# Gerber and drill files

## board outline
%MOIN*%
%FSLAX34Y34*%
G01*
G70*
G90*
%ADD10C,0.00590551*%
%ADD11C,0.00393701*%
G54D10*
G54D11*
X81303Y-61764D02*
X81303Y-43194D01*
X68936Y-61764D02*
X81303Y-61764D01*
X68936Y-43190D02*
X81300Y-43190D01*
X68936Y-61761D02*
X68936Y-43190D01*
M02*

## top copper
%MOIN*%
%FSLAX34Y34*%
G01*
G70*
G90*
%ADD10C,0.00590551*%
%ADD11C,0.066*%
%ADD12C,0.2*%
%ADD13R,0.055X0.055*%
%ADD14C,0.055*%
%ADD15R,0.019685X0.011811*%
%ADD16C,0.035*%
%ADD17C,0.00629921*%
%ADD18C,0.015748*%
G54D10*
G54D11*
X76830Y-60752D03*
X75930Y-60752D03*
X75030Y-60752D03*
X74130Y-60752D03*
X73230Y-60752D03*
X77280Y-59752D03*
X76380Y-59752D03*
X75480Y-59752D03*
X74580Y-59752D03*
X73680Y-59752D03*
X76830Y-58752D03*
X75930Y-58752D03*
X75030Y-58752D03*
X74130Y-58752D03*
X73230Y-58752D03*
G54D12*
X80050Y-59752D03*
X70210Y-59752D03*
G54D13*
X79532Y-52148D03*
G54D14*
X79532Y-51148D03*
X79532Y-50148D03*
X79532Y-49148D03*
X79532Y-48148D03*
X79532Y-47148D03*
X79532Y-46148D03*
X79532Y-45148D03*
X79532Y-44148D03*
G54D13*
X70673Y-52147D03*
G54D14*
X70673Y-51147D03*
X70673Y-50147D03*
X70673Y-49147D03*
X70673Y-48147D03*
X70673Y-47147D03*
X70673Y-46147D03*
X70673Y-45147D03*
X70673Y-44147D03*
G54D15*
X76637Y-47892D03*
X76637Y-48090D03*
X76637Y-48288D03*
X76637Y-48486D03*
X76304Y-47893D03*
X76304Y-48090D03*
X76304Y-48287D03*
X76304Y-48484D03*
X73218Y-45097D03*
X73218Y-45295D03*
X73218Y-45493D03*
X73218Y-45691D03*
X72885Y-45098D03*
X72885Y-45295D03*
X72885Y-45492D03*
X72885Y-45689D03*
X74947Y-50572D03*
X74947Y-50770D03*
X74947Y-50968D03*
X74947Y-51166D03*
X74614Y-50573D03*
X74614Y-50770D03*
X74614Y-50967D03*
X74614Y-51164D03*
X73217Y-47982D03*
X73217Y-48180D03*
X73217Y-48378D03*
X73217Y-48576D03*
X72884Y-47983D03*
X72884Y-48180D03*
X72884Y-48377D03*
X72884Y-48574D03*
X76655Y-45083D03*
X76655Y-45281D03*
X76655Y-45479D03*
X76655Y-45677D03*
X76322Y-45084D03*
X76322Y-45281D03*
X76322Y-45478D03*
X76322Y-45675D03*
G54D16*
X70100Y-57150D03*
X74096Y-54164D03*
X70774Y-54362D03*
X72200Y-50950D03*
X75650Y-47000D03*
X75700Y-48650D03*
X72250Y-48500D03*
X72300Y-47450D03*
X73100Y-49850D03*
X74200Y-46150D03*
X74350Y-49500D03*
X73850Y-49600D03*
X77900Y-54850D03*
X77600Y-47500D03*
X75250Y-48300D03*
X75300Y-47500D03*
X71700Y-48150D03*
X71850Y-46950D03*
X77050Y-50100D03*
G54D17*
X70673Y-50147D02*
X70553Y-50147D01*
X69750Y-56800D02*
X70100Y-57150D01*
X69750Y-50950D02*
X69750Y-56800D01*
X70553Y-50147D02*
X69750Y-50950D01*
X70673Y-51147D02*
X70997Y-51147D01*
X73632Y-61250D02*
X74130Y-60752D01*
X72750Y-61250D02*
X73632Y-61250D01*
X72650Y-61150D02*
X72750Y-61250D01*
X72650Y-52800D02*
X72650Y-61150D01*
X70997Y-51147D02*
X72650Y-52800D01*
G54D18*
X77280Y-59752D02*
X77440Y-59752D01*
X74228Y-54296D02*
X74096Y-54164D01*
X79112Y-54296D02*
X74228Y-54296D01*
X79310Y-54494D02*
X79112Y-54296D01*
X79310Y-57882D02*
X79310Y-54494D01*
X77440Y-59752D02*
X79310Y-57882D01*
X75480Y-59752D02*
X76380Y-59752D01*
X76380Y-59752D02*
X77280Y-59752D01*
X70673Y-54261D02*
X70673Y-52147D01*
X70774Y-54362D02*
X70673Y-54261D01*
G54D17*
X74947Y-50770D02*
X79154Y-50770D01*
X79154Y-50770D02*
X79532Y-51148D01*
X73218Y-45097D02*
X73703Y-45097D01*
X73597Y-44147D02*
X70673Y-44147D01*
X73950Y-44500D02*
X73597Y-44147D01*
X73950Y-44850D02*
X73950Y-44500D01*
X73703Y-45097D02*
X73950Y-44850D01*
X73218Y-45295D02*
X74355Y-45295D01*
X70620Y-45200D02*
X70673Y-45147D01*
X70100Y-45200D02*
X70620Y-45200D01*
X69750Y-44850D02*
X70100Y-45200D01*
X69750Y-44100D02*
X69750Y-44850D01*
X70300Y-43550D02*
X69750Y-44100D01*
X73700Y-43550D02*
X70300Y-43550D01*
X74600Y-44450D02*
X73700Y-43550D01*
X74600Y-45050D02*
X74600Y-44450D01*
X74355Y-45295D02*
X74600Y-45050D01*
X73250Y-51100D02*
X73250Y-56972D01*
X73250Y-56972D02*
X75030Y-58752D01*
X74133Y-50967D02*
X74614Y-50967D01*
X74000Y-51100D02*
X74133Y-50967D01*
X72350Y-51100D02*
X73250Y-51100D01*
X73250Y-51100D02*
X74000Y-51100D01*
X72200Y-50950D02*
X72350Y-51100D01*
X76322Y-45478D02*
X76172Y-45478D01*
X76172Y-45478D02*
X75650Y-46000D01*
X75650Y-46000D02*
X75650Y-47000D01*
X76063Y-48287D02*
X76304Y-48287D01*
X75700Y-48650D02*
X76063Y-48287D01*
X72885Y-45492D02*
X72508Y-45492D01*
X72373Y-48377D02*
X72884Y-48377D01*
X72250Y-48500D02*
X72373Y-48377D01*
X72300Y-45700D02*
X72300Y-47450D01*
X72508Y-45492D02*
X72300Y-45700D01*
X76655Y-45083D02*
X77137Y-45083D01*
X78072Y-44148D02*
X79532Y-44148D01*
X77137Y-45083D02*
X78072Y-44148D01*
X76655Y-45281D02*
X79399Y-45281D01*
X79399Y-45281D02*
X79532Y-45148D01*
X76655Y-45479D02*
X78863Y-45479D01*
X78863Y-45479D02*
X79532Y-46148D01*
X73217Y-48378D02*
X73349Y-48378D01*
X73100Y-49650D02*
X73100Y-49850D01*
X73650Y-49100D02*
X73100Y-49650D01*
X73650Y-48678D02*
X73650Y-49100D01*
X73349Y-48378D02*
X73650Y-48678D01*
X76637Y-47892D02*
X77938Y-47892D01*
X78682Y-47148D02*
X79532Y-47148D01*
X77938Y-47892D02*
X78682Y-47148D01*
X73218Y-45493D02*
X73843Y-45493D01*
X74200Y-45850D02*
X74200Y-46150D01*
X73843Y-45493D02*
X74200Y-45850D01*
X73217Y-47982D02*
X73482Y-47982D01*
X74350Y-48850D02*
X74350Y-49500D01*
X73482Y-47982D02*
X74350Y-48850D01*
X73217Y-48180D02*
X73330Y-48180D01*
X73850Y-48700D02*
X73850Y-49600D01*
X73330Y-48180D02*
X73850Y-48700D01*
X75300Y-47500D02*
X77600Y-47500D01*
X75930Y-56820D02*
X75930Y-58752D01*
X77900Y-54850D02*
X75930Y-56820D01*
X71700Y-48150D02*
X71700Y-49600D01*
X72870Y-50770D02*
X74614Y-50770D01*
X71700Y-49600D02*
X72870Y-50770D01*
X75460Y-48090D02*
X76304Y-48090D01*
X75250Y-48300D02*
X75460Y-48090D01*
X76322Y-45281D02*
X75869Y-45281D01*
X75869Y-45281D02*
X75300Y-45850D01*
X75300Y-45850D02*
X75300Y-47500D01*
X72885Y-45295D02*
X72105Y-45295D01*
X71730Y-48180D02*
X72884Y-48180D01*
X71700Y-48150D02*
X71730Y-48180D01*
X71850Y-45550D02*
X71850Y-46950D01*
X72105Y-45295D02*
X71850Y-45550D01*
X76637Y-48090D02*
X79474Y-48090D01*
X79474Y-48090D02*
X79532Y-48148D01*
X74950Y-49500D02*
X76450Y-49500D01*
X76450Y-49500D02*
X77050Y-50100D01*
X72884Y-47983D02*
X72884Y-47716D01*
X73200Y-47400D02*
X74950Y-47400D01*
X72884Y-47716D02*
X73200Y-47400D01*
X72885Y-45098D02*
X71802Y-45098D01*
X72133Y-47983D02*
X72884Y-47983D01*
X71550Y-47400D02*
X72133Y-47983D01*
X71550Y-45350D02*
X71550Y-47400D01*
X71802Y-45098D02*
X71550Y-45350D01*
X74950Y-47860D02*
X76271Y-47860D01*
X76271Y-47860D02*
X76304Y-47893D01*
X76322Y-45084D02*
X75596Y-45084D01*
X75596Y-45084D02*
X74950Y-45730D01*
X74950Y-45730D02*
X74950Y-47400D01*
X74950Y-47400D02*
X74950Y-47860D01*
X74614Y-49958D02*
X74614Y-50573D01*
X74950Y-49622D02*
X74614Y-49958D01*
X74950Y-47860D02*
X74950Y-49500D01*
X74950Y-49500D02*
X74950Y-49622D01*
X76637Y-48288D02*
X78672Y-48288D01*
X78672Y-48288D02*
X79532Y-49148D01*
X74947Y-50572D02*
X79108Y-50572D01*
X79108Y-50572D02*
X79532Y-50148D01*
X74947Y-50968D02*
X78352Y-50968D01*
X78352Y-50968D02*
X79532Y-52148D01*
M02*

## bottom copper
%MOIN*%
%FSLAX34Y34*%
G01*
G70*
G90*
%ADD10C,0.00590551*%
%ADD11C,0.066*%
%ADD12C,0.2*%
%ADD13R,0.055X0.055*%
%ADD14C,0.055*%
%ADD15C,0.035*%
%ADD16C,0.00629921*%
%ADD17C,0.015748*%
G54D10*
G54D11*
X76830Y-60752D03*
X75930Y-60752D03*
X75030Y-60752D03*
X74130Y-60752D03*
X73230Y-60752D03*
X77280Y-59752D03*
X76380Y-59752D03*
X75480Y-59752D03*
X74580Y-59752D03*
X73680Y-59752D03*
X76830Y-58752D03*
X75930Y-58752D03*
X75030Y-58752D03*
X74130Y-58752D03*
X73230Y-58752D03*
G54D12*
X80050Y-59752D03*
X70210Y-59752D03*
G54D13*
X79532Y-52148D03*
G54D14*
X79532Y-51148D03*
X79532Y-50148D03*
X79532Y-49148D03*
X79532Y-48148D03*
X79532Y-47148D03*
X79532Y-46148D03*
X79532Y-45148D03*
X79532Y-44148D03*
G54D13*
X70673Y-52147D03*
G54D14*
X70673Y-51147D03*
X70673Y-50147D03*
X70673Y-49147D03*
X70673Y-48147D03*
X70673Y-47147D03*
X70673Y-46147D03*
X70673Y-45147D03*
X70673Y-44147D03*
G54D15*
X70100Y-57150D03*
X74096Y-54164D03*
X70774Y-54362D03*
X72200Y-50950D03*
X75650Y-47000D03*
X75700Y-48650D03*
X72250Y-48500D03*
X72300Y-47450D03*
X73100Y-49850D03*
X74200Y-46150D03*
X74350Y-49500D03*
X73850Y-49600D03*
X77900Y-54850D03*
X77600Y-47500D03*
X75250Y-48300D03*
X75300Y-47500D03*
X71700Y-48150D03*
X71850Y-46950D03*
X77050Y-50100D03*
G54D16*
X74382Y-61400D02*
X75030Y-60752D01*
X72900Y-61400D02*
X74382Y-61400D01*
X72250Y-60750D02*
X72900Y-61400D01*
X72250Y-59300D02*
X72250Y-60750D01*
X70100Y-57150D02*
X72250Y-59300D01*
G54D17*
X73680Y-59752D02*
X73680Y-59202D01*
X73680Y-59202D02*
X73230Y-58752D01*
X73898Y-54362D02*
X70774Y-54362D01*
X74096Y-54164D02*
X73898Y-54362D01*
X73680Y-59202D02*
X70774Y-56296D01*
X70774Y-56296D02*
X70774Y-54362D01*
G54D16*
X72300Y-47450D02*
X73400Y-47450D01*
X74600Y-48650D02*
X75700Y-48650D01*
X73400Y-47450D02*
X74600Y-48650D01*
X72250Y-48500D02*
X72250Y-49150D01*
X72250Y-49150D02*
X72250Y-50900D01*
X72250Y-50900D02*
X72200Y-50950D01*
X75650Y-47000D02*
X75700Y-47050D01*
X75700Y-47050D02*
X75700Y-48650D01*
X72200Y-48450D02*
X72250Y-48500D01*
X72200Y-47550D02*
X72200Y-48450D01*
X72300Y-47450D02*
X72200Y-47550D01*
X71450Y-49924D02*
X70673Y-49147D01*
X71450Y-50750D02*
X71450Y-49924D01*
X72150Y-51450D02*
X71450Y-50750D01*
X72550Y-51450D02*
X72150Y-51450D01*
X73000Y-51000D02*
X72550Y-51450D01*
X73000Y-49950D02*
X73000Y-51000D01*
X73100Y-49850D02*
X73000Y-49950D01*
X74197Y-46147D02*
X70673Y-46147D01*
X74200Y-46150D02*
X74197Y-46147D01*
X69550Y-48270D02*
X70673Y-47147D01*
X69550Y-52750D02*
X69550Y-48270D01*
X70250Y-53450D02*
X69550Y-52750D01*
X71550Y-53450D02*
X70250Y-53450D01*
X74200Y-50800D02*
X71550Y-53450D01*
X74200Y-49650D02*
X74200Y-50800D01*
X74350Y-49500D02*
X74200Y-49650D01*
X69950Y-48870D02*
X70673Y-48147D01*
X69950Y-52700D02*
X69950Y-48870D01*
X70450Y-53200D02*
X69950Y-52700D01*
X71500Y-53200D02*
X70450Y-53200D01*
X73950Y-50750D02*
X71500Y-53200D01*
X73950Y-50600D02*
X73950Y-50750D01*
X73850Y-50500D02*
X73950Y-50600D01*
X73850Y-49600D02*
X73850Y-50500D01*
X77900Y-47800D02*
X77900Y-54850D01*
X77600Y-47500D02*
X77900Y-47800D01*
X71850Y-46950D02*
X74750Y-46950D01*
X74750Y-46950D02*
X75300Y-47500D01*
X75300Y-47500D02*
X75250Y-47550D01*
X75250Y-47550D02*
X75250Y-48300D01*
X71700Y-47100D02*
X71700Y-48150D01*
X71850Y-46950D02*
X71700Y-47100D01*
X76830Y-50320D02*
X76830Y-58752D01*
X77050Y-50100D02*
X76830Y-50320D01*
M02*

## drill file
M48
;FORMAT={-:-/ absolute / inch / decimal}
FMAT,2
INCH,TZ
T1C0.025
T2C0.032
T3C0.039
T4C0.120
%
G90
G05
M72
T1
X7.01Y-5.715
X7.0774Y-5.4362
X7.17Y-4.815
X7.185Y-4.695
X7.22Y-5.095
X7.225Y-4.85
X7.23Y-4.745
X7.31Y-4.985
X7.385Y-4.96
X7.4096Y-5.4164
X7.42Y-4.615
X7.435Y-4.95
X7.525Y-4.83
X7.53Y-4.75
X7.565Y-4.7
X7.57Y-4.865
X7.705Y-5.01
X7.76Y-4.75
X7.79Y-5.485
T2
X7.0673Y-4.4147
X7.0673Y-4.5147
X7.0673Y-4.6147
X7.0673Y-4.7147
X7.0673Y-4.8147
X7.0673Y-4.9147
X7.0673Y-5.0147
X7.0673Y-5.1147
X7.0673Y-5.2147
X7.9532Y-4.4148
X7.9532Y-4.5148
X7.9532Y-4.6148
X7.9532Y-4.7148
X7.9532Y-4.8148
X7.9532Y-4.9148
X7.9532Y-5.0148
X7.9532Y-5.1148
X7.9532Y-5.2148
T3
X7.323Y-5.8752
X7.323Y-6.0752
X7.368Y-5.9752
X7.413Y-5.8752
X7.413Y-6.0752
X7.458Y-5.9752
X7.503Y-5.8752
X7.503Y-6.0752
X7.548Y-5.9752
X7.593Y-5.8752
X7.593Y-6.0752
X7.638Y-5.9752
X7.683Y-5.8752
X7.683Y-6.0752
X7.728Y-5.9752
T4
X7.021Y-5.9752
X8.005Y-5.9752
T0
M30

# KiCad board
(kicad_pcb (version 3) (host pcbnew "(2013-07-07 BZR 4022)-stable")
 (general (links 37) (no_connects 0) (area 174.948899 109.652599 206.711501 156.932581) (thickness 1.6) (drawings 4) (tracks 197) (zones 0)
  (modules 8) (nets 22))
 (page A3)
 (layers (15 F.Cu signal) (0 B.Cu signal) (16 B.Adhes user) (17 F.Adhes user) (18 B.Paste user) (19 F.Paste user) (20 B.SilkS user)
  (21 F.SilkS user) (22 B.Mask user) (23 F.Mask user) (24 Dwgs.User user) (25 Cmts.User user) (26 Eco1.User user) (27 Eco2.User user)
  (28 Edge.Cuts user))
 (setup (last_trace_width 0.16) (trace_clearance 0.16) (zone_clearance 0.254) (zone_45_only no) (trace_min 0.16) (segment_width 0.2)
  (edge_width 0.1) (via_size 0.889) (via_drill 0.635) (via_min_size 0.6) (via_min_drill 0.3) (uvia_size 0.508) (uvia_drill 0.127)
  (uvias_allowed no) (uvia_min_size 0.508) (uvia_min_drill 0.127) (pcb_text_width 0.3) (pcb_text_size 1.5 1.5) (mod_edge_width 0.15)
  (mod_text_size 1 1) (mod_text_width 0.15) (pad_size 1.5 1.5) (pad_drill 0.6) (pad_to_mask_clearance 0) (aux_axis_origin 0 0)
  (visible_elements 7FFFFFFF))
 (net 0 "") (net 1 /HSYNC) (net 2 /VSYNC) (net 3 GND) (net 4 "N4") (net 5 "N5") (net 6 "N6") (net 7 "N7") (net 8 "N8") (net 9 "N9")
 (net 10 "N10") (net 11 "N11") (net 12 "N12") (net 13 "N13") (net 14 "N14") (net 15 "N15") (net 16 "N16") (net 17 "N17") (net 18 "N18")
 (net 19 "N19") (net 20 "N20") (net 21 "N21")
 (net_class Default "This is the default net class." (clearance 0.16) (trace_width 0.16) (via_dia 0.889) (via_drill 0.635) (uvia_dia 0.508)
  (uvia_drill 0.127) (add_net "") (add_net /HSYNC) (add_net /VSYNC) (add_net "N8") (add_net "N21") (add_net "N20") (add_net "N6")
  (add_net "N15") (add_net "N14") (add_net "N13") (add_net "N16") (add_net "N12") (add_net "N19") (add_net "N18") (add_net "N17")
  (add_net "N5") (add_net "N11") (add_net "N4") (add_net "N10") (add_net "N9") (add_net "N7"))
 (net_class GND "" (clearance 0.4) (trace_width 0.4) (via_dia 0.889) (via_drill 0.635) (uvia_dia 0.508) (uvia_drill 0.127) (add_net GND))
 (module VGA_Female (layer F.Cu) (at 190.8302 151.77008)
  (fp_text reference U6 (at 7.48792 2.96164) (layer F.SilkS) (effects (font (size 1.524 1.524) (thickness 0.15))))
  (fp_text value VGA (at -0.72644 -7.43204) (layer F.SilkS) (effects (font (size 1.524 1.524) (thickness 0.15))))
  (pad 11 thru_hole circle (at 4.318 2.54) (size 1.6764 1.6764) (drill 0.9906) (layers *.Cu F.Paste F.SilkS F.Mask))
  (pad 12 thru_hole circle (at 2.032 2.54) (size 1.6764 1.6764) (drill 0.9906) (layers *.Cu F.Paste F.SilkS F.Mask))
  (pad 13 thru_hole circle (at -0.254 2.54) (size 1.6764 1.6764) (drill 0.9906) (layers *.Cu F.Paste F.SilkS F.Mask) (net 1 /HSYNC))
  (pad 14 thru_hole circle (at -2.54 2.54) (size 1.6764 1.6764) (drill 0.9906) (layers *.Cu F.Paste F.SilkS F.Mask) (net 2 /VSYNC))
  (pad 15 thru_hole circle (at -4.826 2.54) (size 1.6764 1.6764) (drill 0.9906) (layers *.Cu F.Paste F.SilkS F.Mask))
  (pad 6 thru_hole circle (at 5.461 0) (size 1.6764 1.6764) (drill 0.9906) (layers *.Cu F.Paste F.SilkS F.Mask) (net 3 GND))
  (pad 7 thru_hole circle (at 3.175 0) (size 1.6764 1.6764) (drill 0.9906) (layers *.Cu F.Paste F.SilkS F.Mask) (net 3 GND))
  (pad 8 thru_hole circle (at 0.889 0) (size 1.6764 1.6764) (drill 0.9906) (layers *.Cu F.Paste F.SilkS F.Mask) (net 3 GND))
  (pad 9 thru_hole circle (at -1.397 0) (size 1.6764 1.6764) (drill 0.9906) (layers *.Cu F.Paste F.SilkS F.Mask))
  (pad 10 thru_hole circle (at -3.683 0) (size 1.6764 1.6764) (drill 0.9906) (layers *.Cu F.Paste F.SilkS F.Mask) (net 3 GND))
  (pad 1 thru_hole circle (at 4.318 -2.54) (size 1.6764 1.6764) (drill 0.9906) (layers *.Cu F.Paste F.SilkS F.Mask) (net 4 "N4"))
  (pad 2 thru_hole circle (at 2.032 -2.54) (size 1.6764 1.6764) (drill 0.9906) (layers *.Cu F.Paste F.SilkS F.Mask) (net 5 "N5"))
  (pad 3 thru_hole circle (at -0.254 -2.54) (size 1.6764 1.6764) (drill 0.9906) (layers *.Cu F.Paste F.SilkS F.Mask) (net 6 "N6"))
  (pad 4 thru_hole circle (at -2.54 -2.54) (size 1.6764 1.6764) (drill 0.9906) (layers *.Cu F.Paste F.SilkS F.Mask))
  (pad 5 thru_hole circle (at -4.826 -2.54) (size 1.6764 1.6764) (drill 0.9906) (layers *.Cu F.Paste F.SilkS F.Mask) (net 3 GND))
  (pad SH1 thru_hole circle (at 12.4968 0) (size 5.08 5.08) (drill 3.048) (layers *.Cu F.Paste F.SilkS F.Mask))
  (pad SH2 thru_hole circle (at -12.4968 0) (size 5.08 5.08) (drill 3.048) (layers *.Cu F.Paste F.SilkS F.Mask)))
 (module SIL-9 (layer F.Cu) (at 202.01128 122.29592 90)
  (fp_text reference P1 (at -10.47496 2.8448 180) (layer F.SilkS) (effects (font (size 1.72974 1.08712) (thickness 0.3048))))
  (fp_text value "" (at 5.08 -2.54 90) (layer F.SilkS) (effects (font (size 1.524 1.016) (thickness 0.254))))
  (pad 1 thru_hole rect (at -10.16 0 90) (size 1.397 1.397) (drill 0.8128) (layers *.Cu *.Mask F.SilkS) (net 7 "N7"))
  (pad 2 thru_hole circle (at -7.62 0 90) (size 1.397 1.397) (drill 0.8128) (layers *.Cu *.Mask F.SilkS) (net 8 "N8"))
  (pad 3 thru_hole circle (at -5.08 0 90) (size 1.397 1.397) (drill 0.8128) (layers *.Cu *.Mask F.SilkS) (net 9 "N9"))
  (pad 4 thru_hole circle (at -2.54 0 90) (size 1.397 1.397) (drill 0.8128) (layers *.Cu *.Mask F.SilkS) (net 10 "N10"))
  (pad 5 thru_hole circle (at 0 0 90) (size 1.397 1.397) (drill 0.8128) (layers *.Cu *.Mask F.SilkS) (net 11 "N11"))
  (pad 6 thru_hole circle (at 2.54 0 90) (size 1.397 1.397) (drill 0.8128) (layers *.Cu *.Mask F.SilkS) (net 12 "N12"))
  (pad 7 thru_hole circle (at 5.08 0 90) (size 1.397 1.397) (drill 0.8128) (layers *.Cu *.Mask F.SilkS) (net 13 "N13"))
  (pad 8 thru_hole circle (at 7.62 0 90) (size 1.397 1.397) (drill 0.8128) (layers *.Cu *.Mask F.SilkS) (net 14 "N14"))
  (pad 9 thru_hole circle (at 10.16 0 90) (size 1.397 1.397) (drill 0.8128) (layers *.Cu *.Mask F.SilkS) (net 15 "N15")))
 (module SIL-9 (layer F.Cu) (at 179.50942 122.29338 90)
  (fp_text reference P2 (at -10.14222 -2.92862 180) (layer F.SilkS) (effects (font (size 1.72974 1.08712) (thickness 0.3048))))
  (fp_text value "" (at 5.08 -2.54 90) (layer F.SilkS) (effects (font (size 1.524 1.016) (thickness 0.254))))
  (pad 1 thru_hole rect (at -10.16 0 90) (size 1.397 1.397) (drill 0.8128) (layers *.Cu *.Mask F.SilkS) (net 3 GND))
  (pad 2 thru_hole circle (at -7.62 0 90) (size 1.397 1.397) (drill 0.8128) (layers *.Cu *.Mask F.SilkS) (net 2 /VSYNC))
  (pad 3 thru_hole circle (at -5.08 0 90) (size 1.397 1.397) (drill 0.8128) (layers *.Cu *.Mask F.SilkS) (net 1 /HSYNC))
  (pad 4 thru_hole circle (at -2.54 0 90) (size 1.397 1.397) (drill 0.8128) (layers *.Cu *.Mask F.SilkS) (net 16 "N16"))
  (pad 5 thru_hole circle (at 0 0 90) (size 1.397 1.397) (drill 0.8128) (layers *.Cu *.Mask F.SilkS) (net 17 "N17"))
  (pad 6 thru_hole circle (at 2.54 0 90) (size 1.397 1.397) (drill 0.8128) (layers *.Cu *.Mask F.SilkS) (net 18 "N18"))
  (pad 7 thru_hole circle (at 5.08 0 90) (size 1.397 1.397) (drill 0.8128) (layers *.Cu *.Mask F.SilkS) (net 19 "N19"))
  (pad 8 thru_hole circle (at 7.62 0 90) (size 1.397 1.397) (drill 0.8128) (layers *.Cu *.Mask F.SilkS) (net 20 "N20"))
  (pad 9 thru_hole circle (at 10.16 0 90) (size 1.397 1.397) (drill 0.8128) (layers *.Cu *.Mask F.SilkS) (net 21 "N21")))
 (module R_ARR (layer F.Cu) (at 195.6943 122.3137 270)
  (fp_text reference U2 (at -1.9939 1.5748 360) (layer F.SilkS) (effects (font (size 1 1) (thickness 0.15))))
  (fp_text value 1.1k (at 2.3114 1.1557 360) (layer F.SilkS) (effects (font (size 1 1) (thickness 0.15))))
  (pad 1 smd rect (at -0.66802 1.03632 90) (size 0.3 0.5) (layers F.Cu F.Paste F.Mask) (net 12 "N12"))
  (pad 2 smd rect (at -0.1651 1.03632 90) (size 0.3 0.5) (layers F.Cu F.Paste F.Mask) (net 11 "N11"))
  (pad 3 smd rect (at 0.33782 1.03632 90) (size 0.3 0.5) (layers F.Cu F.Paste F.Mask) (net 10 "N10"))
  (pad 4 smd rect (at 0.84074 1.03632 90) (size 0.3 0.5) (layers F.Cu F.Paste F.Mask))
  (pad 5 smd rect (at -0.66548 1.88214 90) (size 0.3 0.5) (layers F.Cu F.Paste F.Mask) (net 4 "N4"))
  (pad 6 smd rect (at -0.1651 1.88214 90) (size 0.3 0.5) (layers F.Cu F.Paste F.Mask) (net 5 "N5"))
  (pad 7 smd rect (at 0.33528 1.88214 90) (size 0.3 0.5) (layers F.Cu F.Paste F.Mask) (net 6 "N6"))
  (pad 8 smd rect (at 0.83566 1.88214 90) (size 0.3 0.5) (layers F.Cu F.Paste F.Mask)))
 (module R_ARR (layer F.Cu) (at 187.01004 115.2144 270)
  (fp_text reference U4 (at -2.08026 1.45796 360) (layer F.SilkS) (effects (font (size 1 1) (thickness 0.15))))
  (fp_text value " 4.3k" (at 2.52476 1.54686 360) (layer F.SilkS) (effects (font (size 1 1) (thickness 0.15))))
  (pad 1 smd rect (at -0.66802 1.03632 90) (size 0.3 0.5) (layers F.Cu F.Paste F.Mask) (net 21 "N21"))
  (pad 2 smd rect (at -0.1651 1.03632 90) (size 0.3 0.5) (layers F.Cu F.Paste F.Mask) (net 20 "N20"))
  (pad 3 smd rect (at 0.33782 1.03632 90) (size 0.3 0.5) (layers F.Cu F.Paste F.Mask) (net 19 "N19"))
  (pad 4 smd rect (at 0.84074 1.03632 90) (size 0.3 0.5) (layers F.Cu F.Paste F.Mask))
  (pad 5 smd rect (at -0.66548 1.88214 90) (size 0.3 0.5) (layers F.Cu F.Paste F.Mask) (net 4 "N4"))
  (pad 6 smd rect (at -0.1651 1.88214 90) (size 0.3 0.5) (layers F.Cu F.Paste F.Mask) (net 5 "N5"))
  (pad 7 smd rect (at 0.33528 1.88214 90) (size 0.3 0.5) (layers F.Cu F.Paste F.Mask) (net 6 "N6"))
  (pad 8 smd rect (at 0.83566 1.88214 90) (size 0.3 0.5) (layers F.Cu F.Paste F.Mask)))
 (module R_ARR (layer F.Cu) (at 191.4017 129.1209 270)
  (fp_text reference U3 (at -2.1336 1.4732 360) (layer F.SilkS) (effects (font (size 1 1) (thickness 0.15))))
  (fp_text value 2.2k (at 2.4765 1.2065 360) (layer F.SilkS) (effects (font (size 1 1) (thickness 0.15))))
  (pad 1 smd rect (at -0.66802 1.03632 90) (size 0.3 0.5) (layers F.Cu F.Paste F.Mask) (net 9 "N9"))
  (pad 2 smd rect (at -0.1651 1.03632 90) (size 0.3 0.5) (layers F.Cu F.Paste F.Mask) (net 8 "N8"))
  (pad 3 smd rect (at 0.33782 1.03632 90) (size 0.3 0.5) (layers F.Cu F.Paste F.Mask) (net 7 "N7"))
  (pad 4 smd rect (at 0.84074 1.03632 90) (size 0.3 0.5) (layers F.Cu F.Paste F.Mask))
  (pad 5 smd rect (at -0.66548 1.88214 90) (size 0.3 0.5) (layers F.Cu F.Paste F.Mask) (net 4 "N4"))
  (pad 6 smd rect (at -0.1651 1.88214 90) (size 0.3 0.5) (layers F.Cu F.Paste F.Mask) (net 5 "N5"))
  (pad 7 smd rect (at 0.33528 1.88214 90) (size 0.3 0.5) (layers F.Cu F.Paste F.Mask) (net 6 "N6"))
  (pad 8 smd rect (at 0.83566 1.88214 90) (size 0.3 0.5) (layers F.Cu F.Paste F.Mask)))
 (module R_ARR (layer F.Cu) (at 187.0075 122.5423 270)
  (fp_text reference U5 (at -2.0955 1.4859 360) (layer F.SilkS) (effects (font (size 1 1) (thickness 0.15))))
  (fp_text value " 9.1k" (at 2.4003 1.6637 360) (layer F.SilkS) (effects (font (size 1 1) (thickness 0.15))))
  (pad 1 smd rect (at -0.66802 1.03632 90) (size 0.3 0.5) (layers F.Cu F.Paste F.Mask) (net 18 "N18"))
  (pad 2 smd rect (at -0.1651 1.03632 90) (size 0.3 0.5) (layers F.Cu F.Paste F.Mask) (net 17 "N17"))
  (pad 3 smd rect (at 0.33782 1.03632 90) (size 0.3 0.5) (layers F.Cu F.Paste F.Mask) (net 16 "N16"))
  (pad 4 smd rect (at 0.84074 1.03632 90) (size 0.3 0.5) (layers F.Cu F.Paste F.Mask))
  (pad 5 smd rect (at -0.66548 1.88214 90) (size 0.3 0.5) (layers F.Cu F.Paste F.Mask) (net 4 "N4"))
  (pad 6 smd rect (at -0.1651 1.88214 90) (size 0.3 0.5) (layers F.Cu F.Paste F.Mask) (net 5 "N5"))
  (pad 7 smd rect (at 0.33528 1.88214 90) (size 0.3 0.5) (layers F.Cu F.Paste F.Mask) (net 6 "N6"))
  (pad 8 smd rect (at 0.83566 1.88214 90) (size 0.3 0.5) (layers F.Cu F.Paste F.Mask)))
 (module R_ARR (layer F.Cu) (at 195.74002 115.17884 270)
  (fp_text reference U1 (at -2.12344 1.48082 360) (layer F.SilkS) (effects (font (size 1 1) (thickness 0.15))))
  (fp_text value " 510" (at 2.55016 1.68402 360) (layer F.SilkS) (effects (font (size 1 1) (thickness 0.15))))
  (pad 1 smd rect (at -0.66802 1.03632 90) (size 0.3 0.5) (layers F.Cu F.Paste F.Mask) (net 15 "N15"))
  (pad 2 smd rect (at -0.1651 1.03632 90) (size 0.3 0.5) (layers F.Cu F.Paste F.Mask) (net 14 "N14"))
  (pad 3 smd rect (at 0.33782 1.03632 90) (size 0.3 0.5) (layers F.Cu F.Paste F.Mask) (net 13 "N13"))
  (pad 4 smd rect (at 0.84074 1.03632 90) (size 0.3 0.5) (layers F.Cu F.Paste F.Mask))
  (pad 5 smd rect (at -0.66548 1.88214 90) (size 0.3 0.5) (layers F.Cu F.Paste F.Mask) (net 4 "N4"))
  (pad 6 smd rect (at -0.1651 1.88214 90) (size 0.3 0.5) (layers F.Cu F.Paste F.Mask) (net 5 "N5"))
  (pad 7 smd rect (at 0.33528 1.88214 90) (size 0.3 0.5) (layers F.Cu F.Paste F.Mask) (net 6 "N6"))
  (pad 8 smd rect (at 0.83566 1.88214 90) (size 0.3 0.5) (layers F.Cu F.Paste F.Mask)))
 (gr_line (start 206.50962 156.88056) (end 206.50962 109.71276) (angle 90) (layer Edge.Cuts) (width 0.1))
 (gr_line (start 175.09744 156.88056) (end 206.50962 156.88056) (angle 90) (layer Edge.Cuts) (width 0.1))
 (gr_line (start 175.09744 109.7026) (end 206.502 109.7026) (angle 90) (layer Edge.Cuts) (width 0.1))
 (gr_line (start 175.09744 156.87294) (end 175.09744 109.7026) (angle 90) (layer Edge.Cuts) (width 0.1))
 (segment (start 179.50942 127.37338) (end 179.20462 127.37338) (width 0.16) (layer F.Cu) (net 1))
 (segment (start 188.93028 155.956) (end 190.5762 154.31008) (width 0.16) (layer B.Cu) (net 1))
 (segment (start 185.166 155.956) (end 188.93028 155.956) (width 0.16) (layer B.Cu) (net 1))
 (segment (start 183.515 154.305) (end 185.166 155.956) (width 0.16) (layer B.Cu) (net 1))
 (segment (start 183.515 150.622) (end 183.515 154.305) (width 0.16) (layer B.Cu) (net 1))
 (segment (start 178.054 145.161) (end 183.515 150.622) (width 0.16) (layer B.Cu) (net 1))
 (via (at 178.054 145.161) (size 0.889) (layers F.Cu B.Cu) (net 1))
 (segment (start 177.165 144.272) (end 178.054 145.161) (width 0.16) (layer F.Cu) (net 1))
 (segment (start 177.165 129.413) (end 177.165 144.272) (width 0.16) (layer F.Cu) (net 1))
 (segment (start 179.20462 127.37338) (end 177.165 129.413) (width 0.16) (layer F.Cu) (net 1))
 (segment (start 179.50942 129.91338) (end 180.33238 129.91338) (width 0.16) (layer F.Cu) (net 2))
 (segment (start 187.02528 155.575) (end 188.2902 154.31008) (width 0.16) (layer F.Cu) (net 2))
 (segment (start 184.785 155.575) (end 187.02528 155.575) (width 0.16) (layer F.Cu) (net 2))
 (segment (start 184.531 155.321) (end 184.785 155.575) (width 0.16) (layer F.Cu) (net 2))
 (segment (start 184.531 134.112) (end 184.531 155.321) (width 0.16) (layer F.Cu) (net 2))
 (segment (start 180.33238 129.91338) (end 184.531 134.112) (width 0.16) (layer F.Cu) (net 2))
 (segment (start 187.1472 151.77008) (end 187.1472 150.37308) (width 0.4) (layer B.Cu) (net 3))
 (segment (start 187.1472 150.37308) (end 186.0042 149.23008) (width 0.4) (layer B.Cu) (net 3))
 (segment (start 196.2912 151.77008) (end 196.6976 151.77008) (width 0.4) (layer F.Cu) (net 3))
 (segment (start 187.70092 138.07948) (end 179.76596 138.07948) (width 0.4) (layer B.Cu) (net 3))
 (segment (start 188.20384 137.57656) (end 187.70092 138.07948) (width 0.4) (layer B.Cu) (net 3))
 (via (at 188.20384 137.57656) (size 0.889) (layers F.Cu B.Cu) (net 3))
 (segment (start 188.53912 137.91184) (end 188.20384 137.57656) (width 0.4) (layer F.Cu) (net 3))
 (segment (start 200.94448 137.91184) (end 188.53912 137.91184) (width 0.4) (layer F.Cu) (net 3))
 (segment (start 201.4474 138.41476) (end 200.94448 137.91184) (width 0.4) (layer F.Cu) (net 3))
 (segment (start 201.4474 147.02028) (end 201.4474 138.41476) (width 0.4) (layer F.Cu) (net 3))
 (segment (start 196.6976 151.77008) (end 201.4474 147.02028) (width 0.4) (layer F.Cu) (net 3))
 (segment (start 191.7192 151.77008) (end 194.0052 151.77008) (width 0.4) (layer F.Cu) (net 3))
 (segment (start 194.0052 151.77008) (end 196.2912 151.77008) (width 0.4) (layer F.Cu) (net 3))
 (segment (start 187.1472 150.37308) (end 179.76596 142.99184) (width 0.4) (layer B.Cu) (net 3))
 (segment (start 179.76596 142.99184) (end 179.76596 138.07948) (width 0.4) (layer B.Cu) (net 3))
 (segment (start 179.50942 137.82294) (end 179.50942 132.45338) (width 0.4) (layer F.Cu) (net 3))
 (via (at 179.76596 138.07948) (size 0.889) (layers F.Cu B.Cu) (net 3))
 (segment (start 179.76596 138.07948) (end 179.50942 137.82294) (width 0.4) (layer F.Cu) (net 3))
 (segment (start 190.36538 128.9558) (end 201.05116 128.9558) (width 0.16) (layer F.Cu) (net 8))
 (segment (start 201.05116 128.9558) (end 202.01128 129.91592) (width 0.16) (layer F.Cu) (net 8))
 (segment (start 185.97372 114.54638) (end 187.20562 114.54638) (width 0.16) (layer F.Cu) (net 21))
 (segment (start 186.93638 112.13338) (end 179.50942 112.13338) (width 0.16) (layer F.Cu) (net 21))
 (segment (start 187.833 113.03) (end 186.93638 112.13338) (width 0.16) (layer F.Cu) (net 21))
 (segment (start 187.833 113.919) (end 187.833 113.03) (width 0.16) (layer F.Cu) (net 21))
 (segment (start 187.20562 114.54638) (end 187.833 113.919) (width 0.16) (layer F.Cu) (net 21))
 (segment (start 185.97372 115.0493) (end 188.8617 115.0493) (width 0.16) (layer F.Cu) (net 20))
 (segment (start 179.3748 114.808) (end 179.50942 114.67338) (width 0.16) (layer F.Cu) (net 20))
 (segment (start 178.054 114.808) (end 179.3748 114.808) (width 0.16) (layer F.Cu) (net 20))
 (segment (start 177.165 113.919) (end 178.054 114.808) (width 0.16) (layer F.Cu) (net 20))
 (segment (start 177.165 112.014) (end 177.165 113.919) (width 0.16) (layer F.Cu) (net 20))
 (segment (start 178.562 110.617) (end 177.165 112.014) (width 0.16) (layer F.Cu) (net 20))
 (segment (start 187.198 110.617) (end 178.562 110.617) (width 0.16) (layer F.Cu) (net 20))
 (segment (start 189.484 112.903) (end 187.198 110.617) (width 0.16) (layer F.Cu) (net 20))
 (segment (start 189.484 114.427) (end 189.484 112.903) (width 0.16) (layer F.Cu) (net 20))
 (segment (start 188.8617 115.0493) (end 189.484 114.427) (width 0.16) (layer F.Cu) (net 20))
 (segment (start 186.055 129.794) (end 186.055 144.70888) (width 0.16) (layer F.Cu) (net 6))
 (segment (start 186.055 144.70888) (end 190.5762 149.23008) (width 0.16) (layer F.Cu) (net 6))
 (segment (start 183.642 120.523) (end 186.436 120.523) (width 0.16) (layer B.Cu) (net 6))
 (segment (start 189.484 123.571) (end 192.278 123.571) (width 0.16) (layer B.Cu) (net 6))
 (segment (start 186.436 120.523) (end 189.484 123.571) (width 0.16) (layer B.Cu) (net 6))
 (segment (start 183.515 123.19) (end 183.515 124.841) (width 0.16) (layer B.Cu) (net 6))
 (segment (start 183.515 124.841) (end 183.515 129.286) (width 0.16) (layer B.Cu) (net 6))
 (segment (start 188.29782 129.45618) (end 189.51956 129.45618) (width 0.16) (layer F.Cu) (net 6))
 (segment (start 187.96 129.794) (end 188.29782 129.45618) (width 0.16) (layer F.Cu) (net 6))
 (segment (start 183.769 129.794) (end 186.055 129.794) (width 0.16) (layer F.Cu) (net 6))
 (segment (start 186.055 129.794) (end 187.96 129.794) (width 0.16) (layer F.Cu) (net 6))
 (segment (start 183.388 129.413) (end 183.769 129.794) (width 0.16) (layer F.Cu) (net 6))
 (via (at 183.388 129.413) (size 0.889) (layers F.Cu B.Cu) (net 6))
 (segment (start 183.515 129.286) (end 183.388 129.413) (width 0.16) (layer B.Cu) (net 6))
 (segment (start 193.85788 115.51412) (end 193.47688 115.51412) (width 0.16) (layer F.Cu) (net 6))
 (segment (start 193.47688 115.51412) (end 192.151 116.84) (width 0.16) (layer F.Cu) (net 6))
 (segment (start 192.151 116.84) (end 192.151 119.38) (width 0.16) (layer F.Cu) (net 6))
 (via (at 192.151 119.38) (size 0.889) (layers F.Cu B.Cu) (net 6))
 (segment (start 192.151 119.38) (end 192.278 119.507) (width 0.16) (layer B.Cu) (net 6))
 (segment (start 192.278 119.507) (end 192.278 123.571) (width 0.16) (layer B.Cu) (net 6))
 (segment (start 193.20002 122.64898) (end 193.81216 122.64898) (width 0.16) (layer F.Cu) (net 6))
 (via (at 192.278 123.571) (size 0.889) (layers F.Cu B.Cu) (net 6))
 (segment (start 192.278 123.571) (end 193.20002 122.64898) (width 0.16) (layer F.Cu) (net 6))
 (segment (start 185.1279 115.54968) (end 184.17032 115.54968) (width 0.16) (layer F.Cu) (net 6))
 (segment (start 183.82742 122.87758) (end 185.12536 122.87758) (width 0.16) (layer F.Cu) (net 6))
 (segment (start 183.515 123.19) (end 183.82742 122.87758) (width 0.16) (layer F.Cu) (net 6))
 (via (at 183.515 123.19) (size 0.889) (layers F.Cu B.Cu) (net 6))
 (segment (start 183.388 123.063) (end 183.515 123.19) (width 0.16) (layer B.Cu) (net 6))
 (segment (start 183.388 120.777) (end 183.388 123.063) (width 0.16) (layer B.Cu) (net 6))
 (segment (start 183.642 120.523) (end 183.388 120.777) (width 0.16) (layer B.Cu) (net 6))
 (via (at 183.642 120.523) (size 0.889) (layers F.Cu B.Cu) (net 6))
 (segment (start 183.642 116.078) (end 183.642 120.523) (width 0.16) (layer F.Cu) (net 6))
 (segment (start 184.17032 115.54968) (end 183.642 116.078) (width 0.16) (layer F.Cu) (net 6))
 (segment (start 194.7037 114.51082) (end 195.92798 114.51082) (width 0.16) (layer F.Cu) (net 15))
 (segment (start 198.30288 112.13592) (end 202.01128 112.13592) (width 0.16) (layer F.Cu) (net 15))
 (segment (start 195.92798 114.51082) (end 198.30288 112.13592) (width 0.16) (layer F.Cu) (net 15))
 (segment (start 194.7037 115.01374) (end 201.67346 115.01374) (width 0.16) (layer F.Cu) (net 14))
 (segment (start 201.67346 115.01374) (end 202.01128 114.67592) (width 0.16) (layer F.Cu) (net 14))
 (segment (start 194.7037 115.51666) (end 200.31202 115.51666) (width 0.16) (layer F.Cu) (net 13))
 (segment (start 200.31202 115.51666) (end 202.01128 117.21592) (width 0.16) (layer F.Cu) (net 13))
 (segment (start 185.97118 122.88012) (end 186.308568 122.88012) (width 0.16) (layer F.Cu) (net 16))
 (segment (start 181.483 126.80696) (end 179.50942 124.83338) (width 0.16) (layer B.Cu) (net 16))
 (segment (start 181.483 128.905) (end 181.483 126.80696) (width 0.16) (layer B.Cu) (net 16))
 (segment (start 183.261 130.683) (end 181.483 128.905) (width 0.16) (layer B.Cu) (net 16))
 (segment (start 184.277 130.683) (end 183.261 130.683) (width 0.16) (layer B.Cu) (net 16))
 (segment (start 185.42 129.54) (end 184.277 130.683) (width 0.16) (layer B.Cu) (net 16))
 (segment (start 185.42 126.873) (end 185.42 129.54) (width 0.16) (layer B.Cu) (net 16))
 (segment (start 185.674 126.619) (end 185.42 126.873) (width 0.16) (layer B.Cu) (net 16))
 (via (at 185.674 126.619) (size 0.889) (layers F.Cu B.Cu) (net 16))
 (segment (start 185.674 126.111) (end 185.674 126.619) (width 0.16) (layer F.Cu) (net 16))
 (segment (start 187.071 124.714) (end 185.674 126.111) (width 0.16) (layer F.Cu) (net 16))
 (segment (start 187.071 123.642552) (end 187.071 124.714) (width 0.16) (layer F.Cu) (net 16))
 (segment (start 186.308568 122.88012) (end 187.071 123.642552) (width 0.16) (layer F.Cu) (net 16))
 (segment (start 194.65798 121.64568) (end 197.96252 121.64568) (width 0.16) (layer F.Cu) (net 12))
 (segment (start 199.85228 119.75592) (end 202.01128 119.75592) (width 0.16) (layer F.Cu) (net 12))
 (segment (start 197.96252 121.64568) (end 199.85228 119.75592) (width 0.16) (layer F.Cu) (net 12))
 (segment (start 185.97372 115.55222) (end 187.56122 115.55222) (width 0.16) (layer F.Cu) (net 19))
 (segment (start 188.46038 117.21338) (end 179.50942 117.21338) (width 0.16) (layer B.Cu) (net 19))
 (segment (start 188.468 117.221) (end 188.46038 117.21338) (width 0.16) (layer B.Cu) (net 19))
 (via (at 188.468 117.221) (size 0.889) (layers F.Cu B.Cu) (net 19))
 (segment (start 188.468 116.459) (end 188.468 117.221) (width 0.16) (layer F.Cu) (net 19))
 (segment (start 187.56122 115.55222) (end 188.468 116.459) (width 0.16) (layer F.Cu) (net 19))
 (segment (start 185.97118 121.87428) (end 186.64428 121.87428) (width 0.16) (layer F.Cu) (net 18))
 (segment (start 176.657 122.6058) (end 179.50942 119.75338) (width 0.16) (layer B.Cu) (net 18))
 (segment (start 176.657 133.985) (end 176.657 122.6058) (width 0.16) (layer B.Cu) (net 18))
 (segment (start 178.435 135.763) (end 176.657 133.985) (width 0.16) (layer B.Cu) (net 18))
 (segment (start 181.737 135.763) (end 178.435 135.763) (width 0.16) (layer B.Cu) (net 18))
 (segment (start 188.468 129.032) (end 181.737 135.763) (width 0.16) (layer B.Cu) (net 18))
 (segment (start 188.468 126.111) (end 188.468 129.032) (width 0.16) (layer B.Cu) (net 18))
 (segment (start 188.849 125.73) (end 188.468 126.111) (width 0.16) (layer B.Cu) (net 18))
 (via (at 188.849 125.73) (size 0.889) (layers F.Cu B.Cu) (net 18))
 (segment (start 188.849 124.079) (end 188.849 125.73) (width 0.16) (layer F.Cu) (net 18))
 (segment (start 186.64428 121.87428) (end 188.849 124.079) (width 0.16) (layer F.Cu) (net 18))
 (segment (start 185.97118 122.3772) (end 186.2582 122.3772) (width 0.16) (layer F.Cu) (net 17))
 (segment (start 177.673 124.1298) (end 179.50942 122.29338) (width 0.16) (layer B.Cu) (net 17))
 (segment (start 177.673 133.858) (end 177.673 124.1298) (width 0.16) (layer B.Cu) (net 17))
 (segment (start 178.943 135.128) (end 177.673 133.858) (width 0.16) (layer B.Cu) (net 17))
 (segment (start 181.61 135.128) (end 178.943 135.128) (width 0.16) (layer B.Cu) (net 17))
 (segment (start 187.833 128.905) (end 181.61 135.128) (width 0.16) (layer B.Cu) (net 17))
 (segment (start 187.833 128.524) (end 187.833 128.905) (width 0.16) (layer B.Cu) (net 17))
 (segment (start 187.579 128.27) (end 187.833 128.524) (width 0.16) (layer B.Cu) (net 17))
 (segment (start 187.579 125.984) (end 187.579 128.27) (width 0.16) (layer B.Cu) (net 17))
 (via (at 187.579 125.984) (size 0.889) (layers F.Cu B.Cu) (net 17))
 (segment (start 187.579 123.698) (end 187.579 125.984) (width 0.16) (layer F.Cu) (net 17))
 (segment (start 186.2582 122.3772) (end 187.579 123.698) (width 0.16) (layer F.Cu) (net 17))
 (segment (start 191.262 120.65) (end 197.104 120.65) (width 0.16) (layer F.Cu) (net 5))
 (segment (start 192.8622 144.3228) (end 192.8622 149.23008) (width 0.16) (layer F.Cu) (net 5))
 (segment (start 197.866 139.319) (end 192.8622 144.3228) (width 0.16) (layer F.Cu) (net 5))
 (via (at 197.866 139.319) (size 0.889) (layers F.Cu B.Cu) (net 5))
 (segment (start 197.866 121.412) (end 197.866 139.319) (width 0.16) (layer B.Cu) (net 5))
 (segment (start 197.104 120.65) (end 197.866 121.412) (width 0.16) (layer B.Cu) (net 5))
 (via (at 197.104 120.65) (size 0.889) (layers F.Cu B.Cu) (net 5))
 (segment (start 182.118 122.301) (end 182.118 125.984) (width 0.16) (layer F.Cu) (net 5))
 (segment (start 185.0898 128.9558) (end 189.51956 128.9558) (width 0.16) (layer F.Cu) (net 5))
 (segment (start 182.118 125.984) (end 185.0898 128.9558) (width 0.16) (layer F.Cu) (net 5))
 (segment (start 182.499 119.253) (end 189.865 119.253) (width 0.16) (layer B.Cu) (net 5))
 (segment (start 189.865 119.253) (end 191.262 120.65) (width 0.16) (layer B.Cu) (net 5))
 (segment (start 191.6684 122.1486) (end 193.81216 122.1486) (width 0.16) (layer F.Cu) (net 5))
 (segment (start 191.262 120.65) (end 191.135 120.777) (width 0.16) (layer B.Cu) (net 5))
 (segment (start 191.135 120.777) (end 191.135 122.682) (width 0.16) (layer B.Cu) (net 5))
 (via (at 191.135 122.682) (size 0.889) (layers F.Cu B.Cu) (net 5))
 (segment (start 191.135 122.682) (end 191.6684 122.1486) (width 0.16) (layer F.Cu) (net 5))
 (via (at 191.262 120.65) (size 0.889) (layers F.Cu B.Cu) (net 5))
 (segment (start 193.85788 115.01374) (end 192.70726 115.01374) (width 0.16) (layer F.Cu) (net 5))
 (segment (start 192.70726 115.01374) (end 191.262 116.459) (width 0.16) (layer F.Cu) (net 5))
 (segment (start 191.262 116.459) (end 191.262 120.65) (width 0.16) (layer F.Cu) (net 5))
 (segment (start 185.1279 115.0493) (end 183.1467 115.0493) (width 0.16) (layer F.Cu) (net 5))
 (segment (start 182.1942 122.3772) (end 185.12536 122.3772) (width 0.16) (layer F.Cu) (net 5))
 (segment (start 182.118 122.301) (end 182.1942 122.3772) (width 0.16) (layer F.Cu) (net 5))
 (via (at 182.118 122.301) (size 0.889) (layers F.Cu B.Cu) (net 5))
 (segment (start 182.118 119.634) (end 182.118 122.301) (width 0.16) (layer B.Cu) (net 5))
 (segment (start 182.499 119.253) (end 182.118 119.634) (width 0.16) (layer B.Cu) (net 5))
 (via (at 182.499 119.253) (size 0.889) (layers F.Cu B.Cu) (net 5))
 (segment (start 182.499 115.697) (end 182.499 119.253) (width 0.16) (layer F.Cu) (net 5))
 (segment (start 183.1467 115.0493) (end 182.499 115.697) (width 0.16) (layer F.Cu) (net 5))
 (segment (start 194.65798 122.1486) (end 201.86396 122.1486) (width 0.16) (layer F.Cu) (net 11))
 (segment (start 201.86396 122.1486) (end 202.01128 122.29592) (width 0.16) (layer F.Cu) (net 11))
 (segment (start 190.373 125.73) (end 194.183 125.73) (width 0.16) (layer F.Cu) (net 4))
 (segment (start 195.1482 127.8128) (end 195.1482 149.23008) (width 0.16) (layer B.Cu) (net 4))
 (segment (start 195.707 127.254) (end 195.1482 127.8128) (width 0.16) (layer B.Cu) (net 4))
 (via (at 195.707 127.254) (size 0.889) (layers F.Cu B.Cu) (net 4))
 (segment (start 194.183 125.73) (end 195.707 127.254) (width 0.16) (layer F.Cu) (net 4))
 (segment (start 185.12536 121.87682) (end 185.12536 121.19864) (width 0.16) (layer F.Cu) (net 4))
 (segment (start 185.928 120.396) (end 190.373 120.396) (width 0.16) (layer F.Cu) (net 4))
 (segment (start 185.12536 121.19864) (end 185.928 120.396) (width 0.16) (layer F.Cu) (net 4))
 (segment (start 185.1279 114.54892) (end 182.37708 114.54892) (width 0.16) (layer F.Cu) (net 4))
 (segment (start 183.21782 121.87682) (end 185.12536 121.87682) (width 0.16) (layer F.Cu) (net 4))
 (segment (start 181.737 120.396) (end 183.21782 121.87682) (width 0.16) (layer F.Cu) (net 4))
 (segment (start 181.737 115.189) (end 181.737 120.396) (width 0.16) (layer F.Cu) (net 4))
 (segment (start 182.37708 114.54892) (end 181.737 115.189) (width 0.16) (layer F.Cu) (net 4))
 (segment (start 190.373 121.5644) (end 193.72834 121.5644) (width 0.16) (layer F.Cu) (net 4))
 (segment (start 193.72834 121.5644) (end 193.81216 121.64822) (width 0.16) (layer F.Cu) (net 4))
 (segment (start 193.85788 114.51336) (end 192.01384 114.51336) (width 0.16) (layer F.Cu) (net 4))
 (segment (start 192.01384 114.51336) (end 190.373 116.1542) (width 0.16) (layer F.Cu) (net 4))
 (segment (start 190.373 116.1542) (end 190.373 120.396) (width 0.16) (layer F.Cu) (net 4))
 (segment (start 190.373 120.396) (end 190.373 121.5644) (width 0.16) (layer F.Cu) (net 4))
 (segment (start 189.51956 126.89332) (end 189.51956 128.45542) (width 0.16) (layer F.Cu) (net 4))
 (segment (start 190.373 126.03988) (end 189.51956 126.89332) (width 0.16) (layer F.Cu) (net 4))
 (segment (start 190.373 121.5644) (end 190.373 125.73) (width 0.16) (layer F.Cu) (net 4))
 (segment (start 190.373 125.73) (end 190.373 126.03988) (width 0.16) (layer F.Cu) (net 4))
 (segment (start 194.65798 122.65152) (end 199.82688 122.65152) (width 0.16) (layer F.Cu) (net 10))
 (segment (start 199.82688 122.65152) (end 202.01128 124.83592) (width 0.16) (layer F.Cu) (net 10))
 (segment (start 190.36538 128.45288) (end 200.93432 128.45288) (width 0.16) (layer F.Cu) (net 9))
 (segment (start 200.93432 128.45288) (end 202.01128 127.37592) (width 0.16) (layer F.Cu) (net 9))
 (segment (start 190.36538 129.45872) (end 199.01408 129.45872) (width 0.16) (layer F.Cu) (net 7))
 (segment (start 199.01408 129.45872) (end 202.01128 132.45592) (width 0.16) (layer F.Cu) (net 7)))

